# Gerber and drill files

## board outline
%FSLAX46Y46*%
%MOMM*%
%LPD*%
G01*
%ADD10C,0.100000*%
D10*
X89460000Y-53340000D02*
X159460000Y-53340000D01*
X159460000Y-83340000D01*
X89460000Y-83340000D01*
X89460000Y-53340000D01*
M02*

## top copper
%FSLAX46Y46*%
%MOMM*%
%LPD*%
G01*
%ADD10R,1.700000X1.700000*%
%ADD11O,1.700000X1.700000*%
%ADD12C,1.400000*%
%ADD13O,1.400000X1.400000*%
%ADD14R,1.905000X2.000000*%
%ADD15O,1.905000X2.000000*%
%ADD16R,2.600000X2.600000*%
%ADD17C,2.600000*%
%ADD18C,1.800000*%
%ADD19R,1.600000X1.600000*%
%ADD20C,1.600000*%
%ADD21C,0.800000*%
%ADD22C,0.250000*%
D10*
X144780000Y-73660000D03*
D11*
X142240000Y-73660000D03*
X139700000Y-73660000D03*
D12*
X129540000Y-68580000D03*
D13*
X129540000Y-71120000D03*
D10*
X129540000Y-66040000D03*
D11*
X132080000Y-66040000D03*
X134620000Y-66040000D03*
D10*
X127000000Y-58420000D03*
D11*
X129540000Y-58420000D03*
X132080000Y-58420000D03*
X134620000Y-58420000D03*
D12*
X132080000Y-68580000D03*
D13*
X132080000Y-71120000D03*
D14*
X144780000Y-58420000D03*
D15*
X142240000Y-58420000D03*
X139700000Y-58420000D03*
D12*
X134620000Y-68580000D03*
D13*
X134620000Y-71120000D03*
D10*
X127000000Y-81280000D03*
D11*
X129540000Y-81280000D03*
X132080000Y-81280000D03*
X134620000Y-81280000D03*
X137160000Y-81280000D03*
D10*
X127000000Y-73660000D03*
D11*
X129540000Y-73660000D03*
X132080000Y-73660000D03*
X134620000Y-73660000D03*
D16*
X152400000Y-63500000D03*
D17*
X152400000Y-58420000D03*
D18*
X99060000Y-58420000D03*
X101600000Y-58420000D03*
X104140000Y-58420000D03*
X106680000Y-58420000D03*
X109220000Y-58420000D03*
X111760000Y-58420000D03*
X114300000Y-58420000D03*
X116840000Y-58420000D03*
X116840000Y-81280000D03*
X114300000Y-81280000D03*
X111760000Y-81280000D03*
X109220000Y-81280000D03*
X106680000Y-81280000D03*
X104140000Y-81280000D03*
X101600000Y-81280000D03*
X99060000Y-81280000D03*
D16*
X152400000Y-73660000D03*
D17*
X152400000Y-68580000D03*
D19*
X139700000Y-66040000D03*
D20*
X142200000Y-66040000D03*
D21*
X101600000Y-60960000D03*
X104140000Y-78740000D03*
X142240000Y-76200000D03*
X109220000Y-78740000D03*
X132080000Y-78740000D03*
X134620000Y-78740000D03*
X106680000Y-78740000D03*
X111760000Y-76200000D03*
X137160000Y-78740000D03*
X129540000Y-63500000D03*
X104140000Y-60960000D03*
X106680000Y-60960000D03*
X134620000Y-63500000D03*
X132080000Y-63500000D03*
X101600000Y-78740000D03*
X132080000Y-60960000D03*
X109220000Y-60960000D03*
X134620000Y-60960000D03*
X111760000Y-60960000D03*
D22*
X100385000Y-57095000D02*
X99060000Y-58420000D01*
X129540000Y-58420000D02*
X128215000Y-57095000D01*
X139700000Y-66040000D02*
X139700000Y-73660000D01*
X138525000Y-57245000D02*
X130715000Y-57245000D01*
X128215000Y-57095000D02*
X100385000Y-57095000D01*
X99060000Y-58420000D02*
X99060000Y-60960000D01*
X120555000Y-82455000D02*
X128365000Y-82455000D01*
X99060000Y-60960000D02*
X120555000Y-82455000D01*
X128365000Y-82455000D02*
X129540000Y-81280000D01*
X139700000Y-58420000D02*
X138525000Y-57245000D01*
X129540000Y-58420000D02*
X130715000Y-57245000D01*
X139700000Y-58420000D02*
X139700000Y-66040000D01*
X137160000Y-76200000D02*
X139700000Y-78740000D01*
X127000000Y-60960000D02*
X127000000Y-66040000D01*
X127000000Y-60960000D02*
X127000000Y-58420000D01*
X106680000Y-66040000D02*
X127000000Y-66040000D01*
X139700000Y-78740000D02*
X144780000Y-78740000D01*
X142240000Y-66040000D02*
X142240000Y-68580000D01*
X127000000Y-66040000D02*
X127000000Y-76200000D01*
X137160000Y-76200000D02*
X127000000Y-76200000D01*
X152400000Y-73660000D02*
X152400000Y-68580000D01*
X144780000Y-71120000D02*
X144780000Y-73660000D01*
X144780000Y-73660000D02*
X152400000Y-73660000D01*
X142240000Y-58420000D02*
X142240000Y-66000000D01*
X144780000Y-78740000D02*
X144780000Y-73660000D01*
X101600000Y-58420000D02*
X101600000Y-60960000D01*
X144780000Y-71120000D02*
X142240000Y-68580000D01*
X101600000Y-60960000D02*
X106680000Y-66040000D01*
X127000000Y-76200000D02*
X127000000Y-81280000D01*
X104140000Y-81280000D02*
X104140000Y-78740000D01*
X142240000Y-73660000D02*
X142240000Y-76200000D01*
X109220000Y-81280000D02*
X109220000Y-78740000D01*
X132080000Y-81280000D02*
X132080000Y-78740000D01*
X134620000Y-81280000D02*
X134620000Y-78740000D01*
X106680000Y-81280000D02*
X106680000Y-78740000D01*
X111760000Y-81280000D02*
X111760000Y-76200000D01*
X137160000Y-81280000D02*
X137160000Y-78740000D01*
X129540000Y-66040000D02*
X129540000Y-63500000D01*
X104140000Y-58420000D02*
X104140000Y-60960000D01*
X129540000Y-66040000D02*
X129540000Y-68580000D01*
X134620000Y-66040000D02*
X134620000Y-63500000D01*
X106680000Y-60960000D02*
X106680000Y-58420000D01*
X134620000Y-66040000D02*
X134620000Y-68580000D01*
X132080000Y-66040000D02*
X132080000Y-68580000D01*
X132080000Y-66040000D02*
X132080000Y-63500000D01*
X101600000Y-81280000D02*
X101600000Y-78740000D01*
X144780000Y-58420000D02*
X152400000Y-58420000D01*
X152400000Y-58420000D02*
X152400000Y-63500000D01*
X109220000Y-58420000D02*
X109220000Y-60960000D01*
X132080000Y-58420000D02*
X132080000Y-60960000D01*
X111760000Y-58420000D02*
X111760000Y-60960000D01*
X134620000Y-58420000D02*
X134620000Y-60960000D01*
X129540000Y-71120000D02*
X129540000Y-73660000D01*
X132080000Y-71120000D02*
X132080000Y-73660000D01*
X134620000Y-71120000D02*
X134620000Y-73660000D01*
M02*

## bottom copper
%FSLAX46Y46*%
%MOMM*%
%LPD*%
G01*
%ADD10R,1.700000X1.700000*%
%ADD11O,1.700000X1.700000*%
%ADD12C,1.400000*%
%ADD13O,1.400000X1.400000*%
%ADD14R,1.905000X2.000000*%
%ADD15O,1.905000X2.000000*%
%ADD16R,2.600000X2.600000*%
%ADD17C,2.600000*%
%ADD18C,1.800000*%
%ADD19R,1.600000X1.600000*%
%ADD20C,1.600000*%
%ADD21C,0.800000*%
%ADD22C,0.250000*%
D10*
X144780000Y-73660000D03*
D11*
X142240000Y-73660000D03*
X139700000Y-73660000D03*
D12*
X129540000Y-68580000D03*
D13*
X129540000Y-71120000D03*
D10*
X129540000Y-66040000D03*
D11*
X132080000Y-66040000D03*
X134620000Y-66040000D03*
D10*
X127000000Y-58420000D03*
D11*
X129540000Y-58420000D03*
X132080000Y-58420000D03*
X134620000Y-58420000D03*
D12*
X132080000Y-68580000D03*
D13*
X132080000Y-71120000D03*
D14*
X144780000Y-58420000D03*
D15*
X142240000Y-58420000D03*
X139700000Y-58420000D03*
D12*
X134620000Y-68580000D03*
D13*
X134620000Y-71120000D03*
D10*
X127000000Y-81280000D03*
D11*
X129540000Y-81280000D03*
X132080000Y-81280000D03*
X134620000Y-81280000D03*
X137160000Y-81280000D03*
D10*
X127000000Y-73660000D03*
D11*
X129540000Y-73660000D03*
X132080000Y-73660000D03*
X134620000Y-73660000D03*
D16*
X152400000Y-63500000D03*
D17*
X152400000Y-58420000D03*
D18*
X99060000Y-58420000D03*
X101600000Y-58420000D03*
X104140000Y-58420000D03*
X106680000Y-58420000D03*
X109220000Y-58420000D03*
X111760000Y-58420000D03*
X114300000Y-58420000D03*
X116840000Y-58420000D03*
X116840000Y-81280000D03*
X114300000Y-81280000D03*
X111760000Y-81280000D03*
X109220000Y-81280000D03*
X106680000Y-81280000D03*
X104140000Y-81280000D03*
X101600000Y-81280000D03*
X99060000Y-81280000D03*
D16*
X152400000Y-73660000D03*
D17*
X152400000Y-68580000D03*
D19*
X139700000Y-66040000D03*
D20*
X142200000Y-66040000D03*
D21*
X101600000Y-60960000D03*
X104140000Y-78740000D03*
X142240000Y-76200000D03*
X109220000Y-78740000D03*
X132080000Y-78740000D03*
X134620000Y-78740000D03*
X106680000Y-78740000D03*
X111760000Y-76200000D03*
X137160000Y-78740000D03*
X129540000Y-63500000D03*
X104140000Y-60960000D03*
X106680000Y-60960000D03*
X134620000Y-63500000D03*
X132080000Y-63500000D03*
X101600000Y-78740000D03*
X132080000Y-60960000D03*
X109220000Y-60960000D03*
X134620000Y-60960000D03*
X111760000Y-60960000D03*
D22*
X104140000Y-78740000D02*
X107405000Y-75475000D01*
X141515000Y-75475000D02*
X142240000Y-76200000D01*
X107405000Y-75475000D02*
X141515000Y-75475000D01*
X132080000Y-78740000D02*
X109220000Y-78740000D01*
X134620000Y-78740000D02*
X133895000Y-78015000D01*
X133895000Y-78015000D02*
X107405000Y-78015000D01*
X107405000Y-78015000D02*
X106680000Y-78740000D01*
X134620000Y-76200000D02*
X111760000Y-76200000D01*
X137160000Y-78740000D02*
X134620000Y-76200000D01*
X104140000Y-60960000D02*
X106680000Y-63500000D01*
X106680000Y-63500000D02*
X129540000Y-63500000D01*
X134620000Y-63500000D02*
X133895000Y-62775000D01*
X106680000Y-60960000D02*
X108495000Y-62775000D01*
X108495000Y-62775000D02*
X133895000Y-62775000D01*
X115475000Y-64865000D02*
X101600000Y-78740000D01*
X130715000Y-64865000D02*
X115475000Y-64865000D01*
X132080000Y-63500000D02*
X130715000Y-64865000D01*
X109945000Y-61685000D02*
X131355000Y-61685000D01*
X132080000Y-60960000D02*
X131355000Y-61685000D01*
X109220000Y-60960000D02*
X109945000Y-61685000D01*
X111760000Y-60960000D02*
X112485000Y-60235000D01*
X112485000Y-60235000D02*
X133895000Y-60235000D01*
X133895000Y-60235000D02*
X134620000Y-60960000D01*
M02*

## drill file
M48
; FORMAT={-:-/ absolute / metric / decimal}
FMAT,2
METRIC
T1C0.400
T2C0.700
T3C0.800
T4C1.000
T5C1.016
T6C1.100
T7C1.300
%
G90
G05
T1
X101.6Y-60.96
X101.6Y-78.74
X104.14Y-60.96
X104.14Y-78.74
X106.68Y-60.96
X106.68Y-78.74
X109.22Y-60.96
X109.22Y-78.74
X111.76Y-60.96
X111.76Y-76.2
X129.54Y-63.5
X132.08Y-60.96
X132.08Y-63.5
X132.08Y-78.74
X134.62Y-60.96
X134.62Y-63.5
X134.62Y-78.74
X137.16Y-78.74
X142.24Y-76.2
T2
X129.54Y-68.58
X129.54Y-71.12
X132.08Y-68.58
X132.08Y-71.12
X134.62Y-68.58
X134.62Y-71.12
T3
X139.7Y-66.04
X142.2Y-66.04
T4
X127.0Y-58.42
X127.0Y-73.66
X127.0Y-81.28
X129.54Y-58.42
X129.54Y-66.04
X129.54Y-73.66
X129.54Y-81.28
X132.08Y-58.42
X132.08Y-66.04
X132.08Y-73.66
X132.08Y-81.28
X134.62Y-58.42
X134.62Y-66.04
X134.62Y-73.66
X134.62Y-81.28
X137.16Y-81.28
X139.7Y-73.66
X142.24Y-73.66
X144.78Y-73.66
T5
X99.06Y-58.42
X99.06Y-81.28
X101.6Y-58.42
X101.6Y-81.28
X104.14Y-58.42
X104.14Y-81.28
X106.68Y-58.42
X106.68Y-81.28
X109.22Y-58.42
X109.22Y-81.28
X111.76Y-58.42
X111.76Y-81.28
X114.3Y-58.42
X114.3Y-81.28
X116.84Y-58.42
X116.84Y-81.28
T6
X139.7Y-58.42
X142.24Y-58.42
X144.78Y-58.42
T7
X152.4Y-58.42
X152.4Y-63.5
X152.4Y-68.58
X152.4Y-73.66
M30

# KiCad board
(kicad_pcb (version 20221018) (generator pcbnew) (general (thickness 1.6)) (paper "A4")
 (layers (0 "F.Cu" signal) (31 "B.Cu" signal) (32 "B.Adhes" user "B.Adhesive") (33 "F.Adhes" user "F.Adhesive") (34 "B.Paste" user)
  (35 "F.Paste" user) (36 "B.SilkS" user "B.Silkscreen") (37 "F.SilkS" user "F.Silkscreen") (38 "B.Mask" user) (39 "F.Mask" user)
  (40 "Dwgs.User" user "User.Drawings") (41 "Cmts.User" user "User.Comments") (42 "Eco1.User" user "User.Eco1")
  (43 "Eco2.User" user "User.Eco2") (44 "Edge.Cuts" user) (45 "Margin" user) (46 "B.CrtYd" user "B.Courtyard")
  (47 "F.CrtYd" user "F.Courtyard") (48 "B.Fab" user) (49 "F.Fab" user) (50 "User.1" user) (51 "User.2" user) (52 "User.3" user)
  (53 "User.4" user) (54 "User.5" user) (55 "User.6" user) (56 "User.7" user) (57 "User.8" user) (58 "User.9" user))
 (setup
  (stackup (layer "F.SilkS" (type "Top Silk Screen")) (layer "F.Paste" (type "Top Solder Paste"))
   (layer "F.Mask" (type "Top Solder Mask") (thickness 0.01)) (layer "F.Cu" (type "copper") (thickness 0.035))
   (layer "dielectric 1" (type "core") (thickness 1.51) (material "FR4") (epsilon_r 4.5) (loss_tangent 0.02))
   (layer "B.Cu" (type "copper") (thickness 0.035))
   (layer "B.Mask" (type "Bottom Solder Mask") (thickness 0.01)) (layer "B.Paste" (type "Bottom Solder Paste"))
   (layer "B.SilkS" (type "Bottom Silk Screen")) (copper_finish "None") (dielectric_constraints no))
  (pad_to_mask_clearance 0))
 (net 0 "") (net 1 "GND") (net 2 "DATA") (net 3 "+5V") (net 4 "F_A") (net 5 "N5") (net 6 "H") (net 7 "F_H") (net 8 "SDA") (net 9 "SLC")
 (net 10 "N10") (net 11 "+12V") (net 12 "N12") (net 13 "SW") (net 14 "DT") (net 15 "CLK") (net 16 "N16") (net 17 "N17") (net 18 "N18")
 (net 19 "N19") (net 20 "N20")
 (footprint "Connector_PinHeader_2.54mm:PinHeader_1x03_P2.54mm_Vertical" (layer "F.Cu") (at 144.78 73.66 -90)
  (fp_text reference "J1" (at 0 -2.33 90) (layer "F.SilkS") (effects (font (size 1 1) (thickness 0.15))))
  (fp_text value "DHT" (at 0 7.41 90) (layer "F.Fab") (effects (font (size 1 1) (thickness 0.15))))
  (pad "1" thru_hole rect (at 0 0 270) (size 1.7 1.7) (drill 1) (layers "*.Cu" "*.Mask") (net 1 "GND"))
  (pad "2" thru_hole oval (at 0 2.54 270) (size 1.7 1.7) (drill 1) (layers "*.Cu" "*.Mask") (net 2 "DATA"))
  (pad "3" thru_hole oval (at 0 5.08 270) (size 1.7 1.7) (drill 1) (layers "*.Cu" "*.Mask") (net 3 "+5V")))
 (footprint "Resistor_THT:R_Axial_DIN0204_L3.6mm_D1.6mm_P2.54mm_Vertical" (layer "F.Cu") (at 129.54 68.58 -90)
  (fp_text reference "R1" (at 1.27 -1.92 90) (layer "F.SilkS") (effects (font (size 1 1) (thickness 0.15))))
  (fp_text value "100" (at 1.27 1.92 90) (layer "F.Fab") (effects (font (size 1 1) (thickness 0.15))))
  (pad "1" thru_hole circle (at 0 0 270) (size 1.4 1.4) (drill 0.7) (layers "*.Cu" "*.Mask") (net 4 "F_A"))
  (pad "2" thru_hole oval (at 2.54 0 270) (size 1.4 1.4) (drill 0.7) (layers "*.Cu" "*.Mask") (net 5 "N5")))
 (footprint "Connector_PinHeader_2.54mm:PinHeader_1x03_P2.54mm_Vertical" (layer "F.Cu") (at 129.54 66.04 90)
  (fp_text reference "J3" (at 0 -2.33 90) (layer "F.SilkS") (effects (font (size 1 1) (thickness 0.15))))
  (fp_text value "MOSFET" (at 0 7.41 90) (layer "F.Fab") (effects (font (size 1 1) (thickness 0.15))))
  (pad "1" thru_hole rect (at 0 0 90) (size 1.7 1.7) (drill 1) (layers "*.Cu" "*.Mask") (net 4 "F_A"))
  (pad "2" thru_hole oval (at 0 2.54 90) (size 1.7 1.7) (drill 1) (layers "*.Cu" "*.Mask") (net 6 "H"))
  (pad "3" thru_hole oval (at 0 5.08 90) (size 1.7 1.7) (drill 1) (layers "*.Cu" "*.Mask") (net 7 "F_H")))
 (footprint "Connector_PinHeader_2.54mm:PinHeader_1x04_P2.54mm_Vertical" (layer "F.Cu") (at 127 58.42 90)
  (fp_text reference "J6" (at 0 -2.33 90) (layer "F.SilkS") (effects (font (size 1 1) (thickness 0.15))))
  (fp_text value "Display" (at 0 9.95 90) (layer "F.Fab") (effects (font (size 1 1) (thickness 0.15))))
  (pad "1" thru_hole rect (at 0 0 90) (size 1.7 1.7) (drill 1) (layers "*.Cu" "*.Mask") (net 1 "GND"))
  (pad "2" thru_hole oval (at 0 2.54 90) (size 1.7 1.7) (drill 1) (layers "*.Cu" "*.Mask") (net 3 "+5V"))
  (pad "3" thru_hole oval (at 0 5.08 90) (size 1.7 1.7) (drill 1) (layers "*.Cu" "*.Mask") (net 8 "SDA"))
  (pad "4" thru_hole oval (at 0 7.62 90) (size 1.7 1.7) (drill 1) (layers "*.Cu" "*.Mask") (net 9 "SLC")))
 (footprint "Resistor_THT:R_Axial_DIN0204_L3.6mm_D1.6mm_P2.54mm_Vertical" (layer "F.Cu") (at 132.08 68.58 -90)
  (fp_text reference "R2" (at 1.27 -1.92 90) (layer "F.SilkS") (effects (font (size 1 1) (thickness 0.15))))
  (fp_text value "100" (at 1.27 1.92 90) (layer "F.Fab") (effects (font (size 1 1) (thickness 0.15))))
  (pad "1" thru_hole circle (at 0 0 270) (size 1.4 1.4) (drill 0.7) (layers "*.Cu" "*.Mask") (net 6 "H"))
  (pad "2" thru_hole oval (at 2.54 0 270) (size 1.4 1.4) (drill 0.7) (layers "*.Cu" "*.Mask") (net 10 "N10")))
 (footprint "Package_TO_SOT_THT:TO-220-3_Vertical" (layer "F.Cu") (at 144.78 58.42 180)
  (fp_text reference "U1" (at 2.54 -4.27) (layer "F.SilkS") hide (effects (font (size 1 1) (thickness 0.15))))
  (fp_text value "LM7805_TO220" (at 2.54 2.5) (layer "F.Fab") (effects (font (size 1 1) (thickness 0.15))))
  (pad "1" thru_hole rect (at 0 0 180) (size 1.905 2) (drill 1.1) (layers "*.Cu" "*.Mask") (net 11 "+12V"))
  (pad "2" thru_hole oval (at 2.54 0 180) (size 1.905 2) (drill 1.1) (layers "*.Cu" "*.Mask") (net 1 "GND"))
  (pad "3" thru_hole oval (at 5.08 0 180) (size 1.905 2) (drill 1.1) (layers "*.Cu" "*.Mask") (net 3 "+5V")))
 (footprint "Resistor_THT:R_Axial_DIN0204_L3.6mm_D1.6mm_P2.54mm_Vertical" (layer "F.Cu") (at 134.62 68.58 -90)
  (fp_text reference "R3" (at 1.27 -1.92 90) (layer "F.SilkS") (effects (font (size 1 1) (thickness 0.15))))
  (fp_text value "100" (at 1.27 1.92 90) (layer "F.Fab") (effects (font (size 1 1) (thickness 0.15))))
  (pad "1" thru_hole circle (at 0 0 270) (size 1.4 1.4) (drill 0.7) (layers "*.Cu" "*.Mask") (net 7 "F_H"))
  (pad "2" thru_hole oval (at 2.54 0 270) (size 1.4 1.4) (drill 0.7) (layers "*.Cu" "*.Mask") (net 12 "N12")))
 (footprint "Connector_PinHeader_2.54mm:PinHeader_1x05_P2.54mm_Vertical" (layer "F.Cu") (at 127 81.28 90)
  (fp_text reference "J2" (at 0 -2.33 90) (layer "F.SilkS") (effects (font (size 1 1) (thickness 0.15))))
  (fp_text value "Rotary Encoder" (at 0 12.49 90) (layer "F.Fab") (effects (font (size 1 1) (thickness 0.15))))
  (pad "1" thru_hole rect (at 0 0 90) (size 1.7 1.7) (drill 1) (layers "*.Cu" "*.Mask") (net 1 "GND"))
  (pad "2" thru_hole oval (at 0 2.54 90) (size 1.7 1.7) (drill 1) (layers "*.Cu" "*.Mask") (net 3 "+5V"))
  (pad "3" thru_hole oval (at 0 5.08 90) (size 1.7 1.7) (drill 1) (layers "*.Cu" "*.Mask") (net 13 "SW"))
  (pad "4" thru_hole oval (at 0 7.62 90) (size 1.7 1.7) (drill 1) (layers "*.Cu" "*.Mask") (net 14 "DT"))
  (pad "5" thru_hole oval (at 0 10.16 90) (size 1.7 1.7) (drill 1) (layers "*.Cu" "*.Mask") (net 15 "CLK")))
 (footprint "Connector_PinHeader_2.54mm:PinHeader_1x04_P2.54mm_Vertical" (layer "F.Cu") (at 127 73.66 90)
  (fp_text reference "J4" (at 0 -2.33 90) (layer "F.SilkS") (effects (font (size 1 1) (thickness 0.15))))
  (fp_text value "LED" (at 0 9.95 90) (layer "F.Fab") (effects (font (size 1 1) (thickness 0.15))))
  (pad "1" thru_hole rect (at 0 0 90) (size 1.7 1.7) (drill 1) (layers "*.Cu" "*.Mask") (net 1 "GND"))
  (pad "2" thru_hole oval (at 0 2.54 90) (size 1.7 1.7) (drill 1) (layers "*.Cu" "*.Mask") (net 5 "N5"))
  (pad "3" thru_hole oval (at 0 5.08 90) (size 1.7 1.7) (drill 1) (layers "*.Cu" "*.Mask") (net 10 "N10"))
  (pad "4" thru_hole oval (at 0 7.62 90) (size 1.7 1.7) (drill 1) (layers "*.Cu" "*.Mask") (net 12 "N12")))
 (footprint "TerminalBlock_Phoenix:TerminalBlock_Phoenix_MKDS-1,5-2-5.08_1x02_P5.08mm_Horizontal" (layer "F.Cu") (at 152.4 63.5 90)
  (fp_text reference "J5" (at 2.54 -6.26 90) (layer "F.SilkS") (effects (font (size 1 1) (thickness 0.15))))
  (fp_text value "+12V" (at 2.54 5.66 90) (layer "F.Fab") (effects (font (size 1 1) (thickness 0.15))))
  (pad "1" thru_hole rect (at 0 0 90) (size 2.6 2.6) (drill 1.3) (layers "*.Cu" "*.Mask") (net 11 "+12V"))
  (pad "2" thru_hole circle (at 5.08 0 90) (size 2.6 2.6) (drill 1.3) (layers "*.Cu" "*.Mask") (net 11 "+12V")))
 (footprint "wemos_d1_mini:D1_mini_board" (layer "F.Cu") (at 106.68 69.85 -90)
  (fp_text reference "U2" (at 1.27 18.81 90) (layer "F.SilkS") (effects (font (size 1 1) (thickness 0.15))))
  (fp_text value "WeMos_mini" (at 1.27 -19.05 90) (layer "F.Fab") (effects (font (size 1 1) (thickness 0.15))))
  (pad "1" thru_hole circle (at -11.43 7.62 270) (size 1.8 1.8) (drill 1.016) (layers "*.Cu" "*.Mask" "F.SilkS") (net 3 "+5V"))
  (pad "2" thru_hole circle (at -11.43 5.08 270) (size 1.8 1.8) (drill 1.016) (layers "*.Cu" "*.Mask" "F.SilkS") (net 1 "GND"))
  (pad "3" thru_hole circle (at -11.43 2.54 270) (size 1.8 1.8) (drill 1.016) (layers "*.Cu" "*.Mask" "F.SilkS") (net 4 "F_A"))
  (pad "4" thru_hole circle (at -11.43 0 270) (size 1.8 1.8) (drill 1.016) (layers "*.Cu" "*.Mask" "F.SilkS") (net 7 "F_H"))
  (pad "5" thru_hole circle (at -11.43 -2.54 270) (size 1.8 1.8) (drill 1.016) (layers "*.Cu" "*.Mask" "F.SilkS") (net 8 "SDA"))
  (pad "6" thru_hole circle (at -11.43 -5.08 270) (size 1.8 1.8) (drill 1.016) (layers "*.Cu" "*.Mask" "F.SilkS") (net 9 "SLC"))
  (pad "7" thru_hole circle (at -11.43 -7.62 270) (size 1.8 1.8) (drill 1.016) (layers "*.Cu" "*.Mask" "F.SilkS") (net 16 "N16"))
  (pad "8" thru_hole circle (at -11.43 -10.16 270) (size 1.8 1.8) (drill 1.016) (layers "*.Cu" "*.Mask" "F.SilkS") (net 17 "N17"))
  (pad "9" thru_hole circle (at 11.43 -10.16 270) (size 1.8 1.8) (drill 1.016) (layers "*.Cu" "*.Mask" "F.SilkS") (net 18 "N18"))
  (pad "10" thru_hole circle (at 11.43 -7.62 270) (size 1.8 1.8) (drill 1.016) (layers "*.Cu" "*.Mask" "F.SilkS") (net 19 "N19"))
  (pad "11" thru_hole circle (at 11.43 -5.08 270) (size 1.8 1.8) (drill 1.016) (layers "*.Cu" "*.Mask" "F.SilkS") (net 15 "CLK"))
  (pad "12" thru_hole circle (at 11.43 -2.54 270) (size 1.8 1.8) (drill 1.016) (layers "*.Cu" "*.Mask" "F.SilkS") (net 13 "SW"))
  (pad "13" thru_hole circle (at 11.43 0 270) (size 1.8 1.8) (drill 1.016) (layers "*.Cu" "*.Mask" "F.SilkS") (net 14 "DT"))
  (pad "14" thru_hole circle (at 11.43 2.54 270) (size 1.8 1.8) (drill 1.016) (layers "*.Cu" "*.Mask" "F.SilkS") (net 2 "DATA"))
  (pad "15" thru_hole circle (at 11.43 5.08 270) (size 1.8 1.8) (drill 1.016) (layers "*.Cu" "*.Mask" "F.SilkS") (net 6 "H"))
  (pad "16" thru_hole circle (at 11.43 7.62 270) (size 1.8 1.8) (drill 1.016) (layers "*.Cu" "*.Mask" "F.SilkS") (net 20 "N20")))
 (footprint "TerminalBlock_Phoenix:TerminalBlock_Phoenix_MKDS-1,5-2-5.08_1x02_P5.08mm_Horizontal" (layer "F.Cu") (at 152.4 73.66 90)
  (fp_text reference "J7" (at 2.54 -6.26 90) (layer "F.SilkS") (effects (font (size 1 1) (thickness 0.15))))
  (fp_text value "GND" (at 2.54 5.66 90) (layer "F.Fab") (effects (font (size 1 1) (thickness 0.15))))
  (pad "1" thru_hole rect (at 0 0 90) (size 2.6 2.6) (drill 1.3) (layers "*.Cu" "*.Mask") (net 1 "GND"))
  (pad "2" thru_hole circle (at 5.08 0 90) (size 2.6 2.6) (drill 1.3) (layers "*.Cu" "*.Mask") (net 1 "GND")))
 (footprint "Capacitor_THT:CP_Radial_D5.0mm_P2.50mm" (layer "F.Cu") (at 139.7 66.04)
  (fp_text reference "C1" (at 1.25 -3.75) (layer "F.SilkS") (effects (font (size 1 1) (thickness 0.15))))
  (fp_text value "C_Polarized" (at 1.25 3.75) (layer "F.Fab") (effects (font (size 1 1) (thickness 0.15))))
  (pad "1" thru_hole rect (at 0 0) (size 1.6 1.6) (drill 0.8) (layers "*.Cu" "*.Mask") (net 3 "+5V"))
  (pad "2" thru_hole circle (at 2.5 0) (size 1.6 1.6) (drill 0.8) (layers "*.Cu" "*.Mask") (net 1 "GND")))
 (gr_rect (start 89.46 53.34) (end 159.46 83.34) (stroke (width 0.1) (type default)) (fill none) (layer "Edge.Cuts"))
 (segment (start 100.385 57.095) (end 99.06 58.42) (width 0.25) (layer "F.Cu") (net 3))
 (segment (start 129.54 58.42) (end 128.215 57.095) (width 0.25) (layer "F.Cu") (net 3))
 (segment (start 139.7 66.04) (end 139.7 73.66) (width 0.25) (layer "F.Cu") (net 3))
 (segment (start 138.525 57.245) (end 130.715 57.245) (width 0.25) (layer "F.Cu") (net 3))
 (segment (start 128.215 57.095) (end 100.385 57.095) (width 0.25) (layer "F.Cu") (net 3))
 (segment (start 99.06 58.42) (end 99.06 60.96) (width 0.25) (layer "F.Cu") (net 3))
 (segment (start 120.555 82.455) (end 128.365 82.455) (width 0.25) (layer "F.Cu") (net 3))
 (segment (start 99.06 60.96) (end 120.555 82.455) (width 0.25) (layer "F.Cu") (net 3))
 (segment (start 128.365 82.455) (end 129.54 81.28) (width 0.25) (layer "F.Cu") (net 3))
 (segment (start 139.7 58.42) (end 138.525 57.245) (width 0.25) (layer "F.Cu") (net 3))
 (segment (start 129.54 58.42) (end 130.715 57.245) (width 0.25) (layer "F.Cu") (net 3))
 (segment (start 139.7 58.42) (end 139.7 66.04) (width 0.25) (layer "F.Cu") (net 3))
 (segment (start 137.16 76.2) (end 139.7 78.74) (width 0.25) (layer "F.Cu") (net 1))
 (segment (start 127 60.96) (end 127 66.04) (width 0.25) (layer "F.Cu") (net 1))
 (segment (start 127 60.96) (end 127 58.42) (width 0.25) (layer "F.Cu") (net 1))
 (segment (start 106.68 66.04) (end 127 66.04) (width 0.25) (layer "F.Cu") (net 1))
 (segment (start 139.7 78.74) (end 144.78 78.74) (width 0.25) (layer "F.Cu") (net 1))
 (segment (start 142.24 66.04) (end 142.24 68.58) (width 0.25) (layer "F.Cu") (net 1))
 (segment (start 127 66.04) (end 127 76.2) (width 0.25) (layer "F.Cu") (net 1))
 (segment (start 137.16 76.2) (end 127 76.2) (width 0.25) (layer "F.Cu") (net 1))
 (segment (start 152.4 73.66) (end 152.4 68.58) (width 0.25) (layer "F.Cu") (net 1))
 (segment (start 144.78 71.12) (end 144.78 73.66) (width 0.25) (layer "F.Cu") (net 1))
 (segment (start 144.78 73.66) (end 152.4 73.66) (width 0.25) (layer "F.Cu") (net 1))
 (segment (start 142.24 58.42) (end 142.24 66) (width 0.25) (layer "F.Cu") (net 1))
 (segment (start 144.78 78.74) (end 144.78 73.66) (width 0.25) (layer "F.Cu") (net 1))
 (segment (start 101.6 58.42) (end 101.6 60.96) (width 0.25) (layer "F.Cu") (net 1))
 (segment (start 144.78 71.12) (end 142.24 68.58) (width 0.25) (layer "F.Cu") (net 1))
 (segment (start 101.6 60.96) (end 106.68 66.04) (width 0.25) (layer "F.Cu") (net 1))
 (segment (start 127 76.2) (end 127 81.28) (width 0.25) (layer "F.Cu") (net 1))
 (via (at 101.6 60.96) (size 0.8) (drill 0.4) (layers "F.Cu" "B.Cu") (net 1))
 (segment (start 104.14 81.28) (end 104.14 78.74) (width 0.25) (layer "F.Cu") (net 2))
 (segment (start 142.24 73.66) (end 142.24 76.2) (width 0.25) (layer "F.Cu") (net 2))
 (via (at 104.14 78.74) (size 0.8) (drill 0.4) (layers "F.Cu" "B.Cu") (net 2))
 (via (at 142.24 76.2) (size 0.8) (drill 0.4) (layers "F.Cu" "B.Cu") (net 2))
 (segment (start 104.14 78.74) (end 107.405 75.475) (width 0.25) (layer "B.Cu") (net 2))
 (segment (start 141.515 75.475) (end 142.24 76.2) (width 0.25) (layer "B.Cu") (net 2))
 (segment (start 107.405 75.475) (end 141.515 75.475) (width 0.25) (layer "B.Cu") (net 2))
 (segment (start 109.22 81.28) (end 109.22 78.74) (width 0.25) (layer "F.Cu") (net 13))
 (segment (start 132.08 81.28) (end 132.08 78.74) (width 0.25) (layer "F.Cu") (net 13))
 (via (at 109.22 78.74) (size 0.8) (drill 0.4) (layers "F.Cu" "B.Cu") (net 13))
 (via (at 132.08 78.74) (size 0.8) (drill 0.4) (layers "F.Cu" "B.Cu") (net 13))
 (segment (start 132.08 78.74) (end 109.22 78.74) (width 0.25) (layer "B.Cu") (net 13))
 (segment (start 134.62 81.28) (end 134.62 78.74) (width 0.25) (layer "F.Cu") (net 14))
 (segment (start 106.68 81.28) (end 106.68 78.74) (width 0.25) (layer "F.Cu") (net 14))
 (via (at 134.62 78.74) (size 0.8) (drill 0.4) (layers "F.Cu" "B.Cu") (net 14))
 (via (at 106.68 78.74) (size 0.8) (drill 0.4) (layers "F.Cu" "B.Cu") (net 14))
 (segment (start 134.62 78.74) (end 133.895 78.015) (width 0.25) (layer "B.Cu") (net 14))
 (segment (start 133.895 78.015) (end 107.405 78.015) (width 0.25) (layer "B.Cu") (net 14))
 (segment (start 107.405 78.015) (end 106.68 78.74) (width 0.25) (layer "B.Cu") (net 14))
 (segment (start 111.76 81.28) (end 111.76 76.2) (width 0.25) (layer "F.Cu") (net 15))
 (segment (start 137.16 81.28) (end 137.16 78.74) (width 0.25) (layer "F.Cu") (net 15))
 (via (at 111.76 76.2) (size 0.8) (drill 0.4) (layers "F.Cu" "B.Cu") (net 15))
 (via (at 137.16 78.74) (size 0.8) (drill 0.4) (layers "F.Cu" "B.Cu") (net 15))
 (segment (start 134.62 76.2) (end 111.76 76.2) (width 0.25) (layer "B.Cu") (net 15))
 (segment (start 137.16 78.74) (end 134.62 76.2) (width 0.25) (layer "B.Cu") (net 15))
 (segment (start 129.54 66.04) (end 129.54 63.5) (width 0.25) (layer "F.Cu") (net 4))
 (segment (start 104.14 58.42) (end 104.14 60.96) (width 0.25) (layer "F.Cu") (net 4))
 (segment (start 129.54 66.04) (end 129.54 68.58) (width 0.25) (layer "F.Cu") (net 4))
 (via (at 129.54 63.5) (size 0.8) (drill 0.4) (layers "F.Cu" "B.Cu") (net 4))
 (via (at 104.14 60.96) (size 0.8) (drill 0.4) (layers "F.Cu" "B.Cu") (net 4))
 (segment (start 104.14 60.96) (end 106.68 63.5) (width 0.25) (layer "B.Cu") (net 4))
 (segment (start 106.68 63.5) (end 129.54 63.5) (width 0.25) (layer "B.Cu") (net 4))
 (segment (start 134.62 66.04) (end 134.62 63.5) (width 0.25) (layer "F.Cu") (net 7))
 (segment (start 106.68 60.96) (end 106.68 58.42) (width 0.25) (layer "F.Cu") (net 7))
 (segment (start 134.62 66.04) (end 134.62 68.58) (width 0.25) (layer "F.Cu") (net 7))
 (via (at 106.68 60.96) (size 0.8) (drill 0.4) (layers "F.Cu" "B.Cu") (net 7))
 (via (at 134.62 63.5) (size 0.8) (drill 0.4) (layers "F.Cu" "B.Cu") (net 7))
 (segment (start 134.62 63.5) (end 133.895 62.775) (width 0.25) (layer "B.Cu") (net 7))
 (segment (start 106.68 60.96) (end 108.495 62.775) (width 0.25) (layer "B.Cu") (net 7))
 (segment (start 108.495 62.775) (end 133.895 62.775) (width 0.25) (layer "B.Cu") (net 7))
 (segment (start 132.08 66.04) (end 132.08 68.58) (width 0.25) (layer "F.Cu") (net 6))
 (segment (start 132.08 66.04) (end 132.08 63.5) (width 0.25) (layer "F.Cu") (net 6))
 (segment (start 101.6 81.28) (end 101.6 78.74) (width 0.25) (layer "F.Cu") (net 6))
 (via (at 132.08 63.5) (size 0.8) (drill 0.4) (layers "F.Cu" "B.Cu") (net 6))
 (via (at 101.6 78.74) (size 0.8) (drill 0.4) (layers "F.Cu" "B.Cu") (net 6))
 (segment (start 115.475 64.865) (end 101.6 78.74) (width 0.25) (layer "B.Cu") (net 6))
 (segment (start 130.715 64.865) (end 115.475 64.865) (width 0.25) (layer "B.Cu") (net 6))
 (segment (start 132.08 63.5) (end 130.715 64.865) (width 0.25) (layer "B.Cu") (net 6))
 (segment (start 144.78 58.42) (end 152.4 58.42) (width 0.25) (layer "F.Cu") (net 11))
 (segment (start 152.4 58.42) (end 152.4 63.5) (width 0.25) (layer "F.Cu") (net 11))
 (segment (start 109.22 58.42) (end 109.22 60.96) (width 0.25) (layer "F.Cu") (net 8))
 (segment (start 132.08 58.42) (end 132.08 60.96) (width 0.25) (layer "F.Cu") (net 8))
 (via (at 132.08 60.96) (size 0.8) (drill 0.4) (layers "F.Cu" "B.Cu") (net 8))
 (via (at 109.22 60.96) (size 0.8) (drill 0.4) (layers "F.Cu" "B.Cu") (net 8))
 (segment (start 109.945 61.685) (end 131.355 61.685) (width 0.25) (layer "B.Cu") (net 8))
 (segment (start 132.08 60.96) (end 131.355 61.685) (width 0.25) (layer "B.Cu") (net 8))
 (segment (start 109.22 60.96) (end 109.945 61.685) (width 0.25) (layer "B.Cu") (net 8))
 (segment (start 111.76 58.42) (end 111.76 60.96) (width 0.25) (layer "F.Cu") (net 9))
 (segment (start 134.62 58.42) (end 134.62 60.96) (width 0.25) (layer "F.Cu") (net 9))
 (via (at 134.62 60.96) (size 0.8) (drill 0.4) (layers "F.Cu" "B.Cu") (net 9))
 (via (at 111.76 60.96) (size 0.8) (drill 0.4) (layers "F.Cu" "B.Cu") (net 9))
 (segment (start 111.76 60.96) (end 112.485 60.235) (width 0.25) (layer "B.Cu") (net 9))
 (segment (start 112.485 60.235) (end 133.895 60.235) (width 0.25) (layer "B.Cu") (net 9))
 (segment (start 133.895 60.235) (end 134.62 60.96) (width 0.25) (layer "B.Cu") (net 9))
 (segment (start 129.54 71.12) (end 129.54 73.66) (width 0.25) (layer "F.Cu") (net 5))
 (segment (start 132.08 71.12) (end 132.08 73.66) (width 0.25) (layer "F.Cu") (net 10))
 (segment (start 134.62 71.12) (end 134.62 73.66) (width 0.25) (layer "F.Cu") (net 12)))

